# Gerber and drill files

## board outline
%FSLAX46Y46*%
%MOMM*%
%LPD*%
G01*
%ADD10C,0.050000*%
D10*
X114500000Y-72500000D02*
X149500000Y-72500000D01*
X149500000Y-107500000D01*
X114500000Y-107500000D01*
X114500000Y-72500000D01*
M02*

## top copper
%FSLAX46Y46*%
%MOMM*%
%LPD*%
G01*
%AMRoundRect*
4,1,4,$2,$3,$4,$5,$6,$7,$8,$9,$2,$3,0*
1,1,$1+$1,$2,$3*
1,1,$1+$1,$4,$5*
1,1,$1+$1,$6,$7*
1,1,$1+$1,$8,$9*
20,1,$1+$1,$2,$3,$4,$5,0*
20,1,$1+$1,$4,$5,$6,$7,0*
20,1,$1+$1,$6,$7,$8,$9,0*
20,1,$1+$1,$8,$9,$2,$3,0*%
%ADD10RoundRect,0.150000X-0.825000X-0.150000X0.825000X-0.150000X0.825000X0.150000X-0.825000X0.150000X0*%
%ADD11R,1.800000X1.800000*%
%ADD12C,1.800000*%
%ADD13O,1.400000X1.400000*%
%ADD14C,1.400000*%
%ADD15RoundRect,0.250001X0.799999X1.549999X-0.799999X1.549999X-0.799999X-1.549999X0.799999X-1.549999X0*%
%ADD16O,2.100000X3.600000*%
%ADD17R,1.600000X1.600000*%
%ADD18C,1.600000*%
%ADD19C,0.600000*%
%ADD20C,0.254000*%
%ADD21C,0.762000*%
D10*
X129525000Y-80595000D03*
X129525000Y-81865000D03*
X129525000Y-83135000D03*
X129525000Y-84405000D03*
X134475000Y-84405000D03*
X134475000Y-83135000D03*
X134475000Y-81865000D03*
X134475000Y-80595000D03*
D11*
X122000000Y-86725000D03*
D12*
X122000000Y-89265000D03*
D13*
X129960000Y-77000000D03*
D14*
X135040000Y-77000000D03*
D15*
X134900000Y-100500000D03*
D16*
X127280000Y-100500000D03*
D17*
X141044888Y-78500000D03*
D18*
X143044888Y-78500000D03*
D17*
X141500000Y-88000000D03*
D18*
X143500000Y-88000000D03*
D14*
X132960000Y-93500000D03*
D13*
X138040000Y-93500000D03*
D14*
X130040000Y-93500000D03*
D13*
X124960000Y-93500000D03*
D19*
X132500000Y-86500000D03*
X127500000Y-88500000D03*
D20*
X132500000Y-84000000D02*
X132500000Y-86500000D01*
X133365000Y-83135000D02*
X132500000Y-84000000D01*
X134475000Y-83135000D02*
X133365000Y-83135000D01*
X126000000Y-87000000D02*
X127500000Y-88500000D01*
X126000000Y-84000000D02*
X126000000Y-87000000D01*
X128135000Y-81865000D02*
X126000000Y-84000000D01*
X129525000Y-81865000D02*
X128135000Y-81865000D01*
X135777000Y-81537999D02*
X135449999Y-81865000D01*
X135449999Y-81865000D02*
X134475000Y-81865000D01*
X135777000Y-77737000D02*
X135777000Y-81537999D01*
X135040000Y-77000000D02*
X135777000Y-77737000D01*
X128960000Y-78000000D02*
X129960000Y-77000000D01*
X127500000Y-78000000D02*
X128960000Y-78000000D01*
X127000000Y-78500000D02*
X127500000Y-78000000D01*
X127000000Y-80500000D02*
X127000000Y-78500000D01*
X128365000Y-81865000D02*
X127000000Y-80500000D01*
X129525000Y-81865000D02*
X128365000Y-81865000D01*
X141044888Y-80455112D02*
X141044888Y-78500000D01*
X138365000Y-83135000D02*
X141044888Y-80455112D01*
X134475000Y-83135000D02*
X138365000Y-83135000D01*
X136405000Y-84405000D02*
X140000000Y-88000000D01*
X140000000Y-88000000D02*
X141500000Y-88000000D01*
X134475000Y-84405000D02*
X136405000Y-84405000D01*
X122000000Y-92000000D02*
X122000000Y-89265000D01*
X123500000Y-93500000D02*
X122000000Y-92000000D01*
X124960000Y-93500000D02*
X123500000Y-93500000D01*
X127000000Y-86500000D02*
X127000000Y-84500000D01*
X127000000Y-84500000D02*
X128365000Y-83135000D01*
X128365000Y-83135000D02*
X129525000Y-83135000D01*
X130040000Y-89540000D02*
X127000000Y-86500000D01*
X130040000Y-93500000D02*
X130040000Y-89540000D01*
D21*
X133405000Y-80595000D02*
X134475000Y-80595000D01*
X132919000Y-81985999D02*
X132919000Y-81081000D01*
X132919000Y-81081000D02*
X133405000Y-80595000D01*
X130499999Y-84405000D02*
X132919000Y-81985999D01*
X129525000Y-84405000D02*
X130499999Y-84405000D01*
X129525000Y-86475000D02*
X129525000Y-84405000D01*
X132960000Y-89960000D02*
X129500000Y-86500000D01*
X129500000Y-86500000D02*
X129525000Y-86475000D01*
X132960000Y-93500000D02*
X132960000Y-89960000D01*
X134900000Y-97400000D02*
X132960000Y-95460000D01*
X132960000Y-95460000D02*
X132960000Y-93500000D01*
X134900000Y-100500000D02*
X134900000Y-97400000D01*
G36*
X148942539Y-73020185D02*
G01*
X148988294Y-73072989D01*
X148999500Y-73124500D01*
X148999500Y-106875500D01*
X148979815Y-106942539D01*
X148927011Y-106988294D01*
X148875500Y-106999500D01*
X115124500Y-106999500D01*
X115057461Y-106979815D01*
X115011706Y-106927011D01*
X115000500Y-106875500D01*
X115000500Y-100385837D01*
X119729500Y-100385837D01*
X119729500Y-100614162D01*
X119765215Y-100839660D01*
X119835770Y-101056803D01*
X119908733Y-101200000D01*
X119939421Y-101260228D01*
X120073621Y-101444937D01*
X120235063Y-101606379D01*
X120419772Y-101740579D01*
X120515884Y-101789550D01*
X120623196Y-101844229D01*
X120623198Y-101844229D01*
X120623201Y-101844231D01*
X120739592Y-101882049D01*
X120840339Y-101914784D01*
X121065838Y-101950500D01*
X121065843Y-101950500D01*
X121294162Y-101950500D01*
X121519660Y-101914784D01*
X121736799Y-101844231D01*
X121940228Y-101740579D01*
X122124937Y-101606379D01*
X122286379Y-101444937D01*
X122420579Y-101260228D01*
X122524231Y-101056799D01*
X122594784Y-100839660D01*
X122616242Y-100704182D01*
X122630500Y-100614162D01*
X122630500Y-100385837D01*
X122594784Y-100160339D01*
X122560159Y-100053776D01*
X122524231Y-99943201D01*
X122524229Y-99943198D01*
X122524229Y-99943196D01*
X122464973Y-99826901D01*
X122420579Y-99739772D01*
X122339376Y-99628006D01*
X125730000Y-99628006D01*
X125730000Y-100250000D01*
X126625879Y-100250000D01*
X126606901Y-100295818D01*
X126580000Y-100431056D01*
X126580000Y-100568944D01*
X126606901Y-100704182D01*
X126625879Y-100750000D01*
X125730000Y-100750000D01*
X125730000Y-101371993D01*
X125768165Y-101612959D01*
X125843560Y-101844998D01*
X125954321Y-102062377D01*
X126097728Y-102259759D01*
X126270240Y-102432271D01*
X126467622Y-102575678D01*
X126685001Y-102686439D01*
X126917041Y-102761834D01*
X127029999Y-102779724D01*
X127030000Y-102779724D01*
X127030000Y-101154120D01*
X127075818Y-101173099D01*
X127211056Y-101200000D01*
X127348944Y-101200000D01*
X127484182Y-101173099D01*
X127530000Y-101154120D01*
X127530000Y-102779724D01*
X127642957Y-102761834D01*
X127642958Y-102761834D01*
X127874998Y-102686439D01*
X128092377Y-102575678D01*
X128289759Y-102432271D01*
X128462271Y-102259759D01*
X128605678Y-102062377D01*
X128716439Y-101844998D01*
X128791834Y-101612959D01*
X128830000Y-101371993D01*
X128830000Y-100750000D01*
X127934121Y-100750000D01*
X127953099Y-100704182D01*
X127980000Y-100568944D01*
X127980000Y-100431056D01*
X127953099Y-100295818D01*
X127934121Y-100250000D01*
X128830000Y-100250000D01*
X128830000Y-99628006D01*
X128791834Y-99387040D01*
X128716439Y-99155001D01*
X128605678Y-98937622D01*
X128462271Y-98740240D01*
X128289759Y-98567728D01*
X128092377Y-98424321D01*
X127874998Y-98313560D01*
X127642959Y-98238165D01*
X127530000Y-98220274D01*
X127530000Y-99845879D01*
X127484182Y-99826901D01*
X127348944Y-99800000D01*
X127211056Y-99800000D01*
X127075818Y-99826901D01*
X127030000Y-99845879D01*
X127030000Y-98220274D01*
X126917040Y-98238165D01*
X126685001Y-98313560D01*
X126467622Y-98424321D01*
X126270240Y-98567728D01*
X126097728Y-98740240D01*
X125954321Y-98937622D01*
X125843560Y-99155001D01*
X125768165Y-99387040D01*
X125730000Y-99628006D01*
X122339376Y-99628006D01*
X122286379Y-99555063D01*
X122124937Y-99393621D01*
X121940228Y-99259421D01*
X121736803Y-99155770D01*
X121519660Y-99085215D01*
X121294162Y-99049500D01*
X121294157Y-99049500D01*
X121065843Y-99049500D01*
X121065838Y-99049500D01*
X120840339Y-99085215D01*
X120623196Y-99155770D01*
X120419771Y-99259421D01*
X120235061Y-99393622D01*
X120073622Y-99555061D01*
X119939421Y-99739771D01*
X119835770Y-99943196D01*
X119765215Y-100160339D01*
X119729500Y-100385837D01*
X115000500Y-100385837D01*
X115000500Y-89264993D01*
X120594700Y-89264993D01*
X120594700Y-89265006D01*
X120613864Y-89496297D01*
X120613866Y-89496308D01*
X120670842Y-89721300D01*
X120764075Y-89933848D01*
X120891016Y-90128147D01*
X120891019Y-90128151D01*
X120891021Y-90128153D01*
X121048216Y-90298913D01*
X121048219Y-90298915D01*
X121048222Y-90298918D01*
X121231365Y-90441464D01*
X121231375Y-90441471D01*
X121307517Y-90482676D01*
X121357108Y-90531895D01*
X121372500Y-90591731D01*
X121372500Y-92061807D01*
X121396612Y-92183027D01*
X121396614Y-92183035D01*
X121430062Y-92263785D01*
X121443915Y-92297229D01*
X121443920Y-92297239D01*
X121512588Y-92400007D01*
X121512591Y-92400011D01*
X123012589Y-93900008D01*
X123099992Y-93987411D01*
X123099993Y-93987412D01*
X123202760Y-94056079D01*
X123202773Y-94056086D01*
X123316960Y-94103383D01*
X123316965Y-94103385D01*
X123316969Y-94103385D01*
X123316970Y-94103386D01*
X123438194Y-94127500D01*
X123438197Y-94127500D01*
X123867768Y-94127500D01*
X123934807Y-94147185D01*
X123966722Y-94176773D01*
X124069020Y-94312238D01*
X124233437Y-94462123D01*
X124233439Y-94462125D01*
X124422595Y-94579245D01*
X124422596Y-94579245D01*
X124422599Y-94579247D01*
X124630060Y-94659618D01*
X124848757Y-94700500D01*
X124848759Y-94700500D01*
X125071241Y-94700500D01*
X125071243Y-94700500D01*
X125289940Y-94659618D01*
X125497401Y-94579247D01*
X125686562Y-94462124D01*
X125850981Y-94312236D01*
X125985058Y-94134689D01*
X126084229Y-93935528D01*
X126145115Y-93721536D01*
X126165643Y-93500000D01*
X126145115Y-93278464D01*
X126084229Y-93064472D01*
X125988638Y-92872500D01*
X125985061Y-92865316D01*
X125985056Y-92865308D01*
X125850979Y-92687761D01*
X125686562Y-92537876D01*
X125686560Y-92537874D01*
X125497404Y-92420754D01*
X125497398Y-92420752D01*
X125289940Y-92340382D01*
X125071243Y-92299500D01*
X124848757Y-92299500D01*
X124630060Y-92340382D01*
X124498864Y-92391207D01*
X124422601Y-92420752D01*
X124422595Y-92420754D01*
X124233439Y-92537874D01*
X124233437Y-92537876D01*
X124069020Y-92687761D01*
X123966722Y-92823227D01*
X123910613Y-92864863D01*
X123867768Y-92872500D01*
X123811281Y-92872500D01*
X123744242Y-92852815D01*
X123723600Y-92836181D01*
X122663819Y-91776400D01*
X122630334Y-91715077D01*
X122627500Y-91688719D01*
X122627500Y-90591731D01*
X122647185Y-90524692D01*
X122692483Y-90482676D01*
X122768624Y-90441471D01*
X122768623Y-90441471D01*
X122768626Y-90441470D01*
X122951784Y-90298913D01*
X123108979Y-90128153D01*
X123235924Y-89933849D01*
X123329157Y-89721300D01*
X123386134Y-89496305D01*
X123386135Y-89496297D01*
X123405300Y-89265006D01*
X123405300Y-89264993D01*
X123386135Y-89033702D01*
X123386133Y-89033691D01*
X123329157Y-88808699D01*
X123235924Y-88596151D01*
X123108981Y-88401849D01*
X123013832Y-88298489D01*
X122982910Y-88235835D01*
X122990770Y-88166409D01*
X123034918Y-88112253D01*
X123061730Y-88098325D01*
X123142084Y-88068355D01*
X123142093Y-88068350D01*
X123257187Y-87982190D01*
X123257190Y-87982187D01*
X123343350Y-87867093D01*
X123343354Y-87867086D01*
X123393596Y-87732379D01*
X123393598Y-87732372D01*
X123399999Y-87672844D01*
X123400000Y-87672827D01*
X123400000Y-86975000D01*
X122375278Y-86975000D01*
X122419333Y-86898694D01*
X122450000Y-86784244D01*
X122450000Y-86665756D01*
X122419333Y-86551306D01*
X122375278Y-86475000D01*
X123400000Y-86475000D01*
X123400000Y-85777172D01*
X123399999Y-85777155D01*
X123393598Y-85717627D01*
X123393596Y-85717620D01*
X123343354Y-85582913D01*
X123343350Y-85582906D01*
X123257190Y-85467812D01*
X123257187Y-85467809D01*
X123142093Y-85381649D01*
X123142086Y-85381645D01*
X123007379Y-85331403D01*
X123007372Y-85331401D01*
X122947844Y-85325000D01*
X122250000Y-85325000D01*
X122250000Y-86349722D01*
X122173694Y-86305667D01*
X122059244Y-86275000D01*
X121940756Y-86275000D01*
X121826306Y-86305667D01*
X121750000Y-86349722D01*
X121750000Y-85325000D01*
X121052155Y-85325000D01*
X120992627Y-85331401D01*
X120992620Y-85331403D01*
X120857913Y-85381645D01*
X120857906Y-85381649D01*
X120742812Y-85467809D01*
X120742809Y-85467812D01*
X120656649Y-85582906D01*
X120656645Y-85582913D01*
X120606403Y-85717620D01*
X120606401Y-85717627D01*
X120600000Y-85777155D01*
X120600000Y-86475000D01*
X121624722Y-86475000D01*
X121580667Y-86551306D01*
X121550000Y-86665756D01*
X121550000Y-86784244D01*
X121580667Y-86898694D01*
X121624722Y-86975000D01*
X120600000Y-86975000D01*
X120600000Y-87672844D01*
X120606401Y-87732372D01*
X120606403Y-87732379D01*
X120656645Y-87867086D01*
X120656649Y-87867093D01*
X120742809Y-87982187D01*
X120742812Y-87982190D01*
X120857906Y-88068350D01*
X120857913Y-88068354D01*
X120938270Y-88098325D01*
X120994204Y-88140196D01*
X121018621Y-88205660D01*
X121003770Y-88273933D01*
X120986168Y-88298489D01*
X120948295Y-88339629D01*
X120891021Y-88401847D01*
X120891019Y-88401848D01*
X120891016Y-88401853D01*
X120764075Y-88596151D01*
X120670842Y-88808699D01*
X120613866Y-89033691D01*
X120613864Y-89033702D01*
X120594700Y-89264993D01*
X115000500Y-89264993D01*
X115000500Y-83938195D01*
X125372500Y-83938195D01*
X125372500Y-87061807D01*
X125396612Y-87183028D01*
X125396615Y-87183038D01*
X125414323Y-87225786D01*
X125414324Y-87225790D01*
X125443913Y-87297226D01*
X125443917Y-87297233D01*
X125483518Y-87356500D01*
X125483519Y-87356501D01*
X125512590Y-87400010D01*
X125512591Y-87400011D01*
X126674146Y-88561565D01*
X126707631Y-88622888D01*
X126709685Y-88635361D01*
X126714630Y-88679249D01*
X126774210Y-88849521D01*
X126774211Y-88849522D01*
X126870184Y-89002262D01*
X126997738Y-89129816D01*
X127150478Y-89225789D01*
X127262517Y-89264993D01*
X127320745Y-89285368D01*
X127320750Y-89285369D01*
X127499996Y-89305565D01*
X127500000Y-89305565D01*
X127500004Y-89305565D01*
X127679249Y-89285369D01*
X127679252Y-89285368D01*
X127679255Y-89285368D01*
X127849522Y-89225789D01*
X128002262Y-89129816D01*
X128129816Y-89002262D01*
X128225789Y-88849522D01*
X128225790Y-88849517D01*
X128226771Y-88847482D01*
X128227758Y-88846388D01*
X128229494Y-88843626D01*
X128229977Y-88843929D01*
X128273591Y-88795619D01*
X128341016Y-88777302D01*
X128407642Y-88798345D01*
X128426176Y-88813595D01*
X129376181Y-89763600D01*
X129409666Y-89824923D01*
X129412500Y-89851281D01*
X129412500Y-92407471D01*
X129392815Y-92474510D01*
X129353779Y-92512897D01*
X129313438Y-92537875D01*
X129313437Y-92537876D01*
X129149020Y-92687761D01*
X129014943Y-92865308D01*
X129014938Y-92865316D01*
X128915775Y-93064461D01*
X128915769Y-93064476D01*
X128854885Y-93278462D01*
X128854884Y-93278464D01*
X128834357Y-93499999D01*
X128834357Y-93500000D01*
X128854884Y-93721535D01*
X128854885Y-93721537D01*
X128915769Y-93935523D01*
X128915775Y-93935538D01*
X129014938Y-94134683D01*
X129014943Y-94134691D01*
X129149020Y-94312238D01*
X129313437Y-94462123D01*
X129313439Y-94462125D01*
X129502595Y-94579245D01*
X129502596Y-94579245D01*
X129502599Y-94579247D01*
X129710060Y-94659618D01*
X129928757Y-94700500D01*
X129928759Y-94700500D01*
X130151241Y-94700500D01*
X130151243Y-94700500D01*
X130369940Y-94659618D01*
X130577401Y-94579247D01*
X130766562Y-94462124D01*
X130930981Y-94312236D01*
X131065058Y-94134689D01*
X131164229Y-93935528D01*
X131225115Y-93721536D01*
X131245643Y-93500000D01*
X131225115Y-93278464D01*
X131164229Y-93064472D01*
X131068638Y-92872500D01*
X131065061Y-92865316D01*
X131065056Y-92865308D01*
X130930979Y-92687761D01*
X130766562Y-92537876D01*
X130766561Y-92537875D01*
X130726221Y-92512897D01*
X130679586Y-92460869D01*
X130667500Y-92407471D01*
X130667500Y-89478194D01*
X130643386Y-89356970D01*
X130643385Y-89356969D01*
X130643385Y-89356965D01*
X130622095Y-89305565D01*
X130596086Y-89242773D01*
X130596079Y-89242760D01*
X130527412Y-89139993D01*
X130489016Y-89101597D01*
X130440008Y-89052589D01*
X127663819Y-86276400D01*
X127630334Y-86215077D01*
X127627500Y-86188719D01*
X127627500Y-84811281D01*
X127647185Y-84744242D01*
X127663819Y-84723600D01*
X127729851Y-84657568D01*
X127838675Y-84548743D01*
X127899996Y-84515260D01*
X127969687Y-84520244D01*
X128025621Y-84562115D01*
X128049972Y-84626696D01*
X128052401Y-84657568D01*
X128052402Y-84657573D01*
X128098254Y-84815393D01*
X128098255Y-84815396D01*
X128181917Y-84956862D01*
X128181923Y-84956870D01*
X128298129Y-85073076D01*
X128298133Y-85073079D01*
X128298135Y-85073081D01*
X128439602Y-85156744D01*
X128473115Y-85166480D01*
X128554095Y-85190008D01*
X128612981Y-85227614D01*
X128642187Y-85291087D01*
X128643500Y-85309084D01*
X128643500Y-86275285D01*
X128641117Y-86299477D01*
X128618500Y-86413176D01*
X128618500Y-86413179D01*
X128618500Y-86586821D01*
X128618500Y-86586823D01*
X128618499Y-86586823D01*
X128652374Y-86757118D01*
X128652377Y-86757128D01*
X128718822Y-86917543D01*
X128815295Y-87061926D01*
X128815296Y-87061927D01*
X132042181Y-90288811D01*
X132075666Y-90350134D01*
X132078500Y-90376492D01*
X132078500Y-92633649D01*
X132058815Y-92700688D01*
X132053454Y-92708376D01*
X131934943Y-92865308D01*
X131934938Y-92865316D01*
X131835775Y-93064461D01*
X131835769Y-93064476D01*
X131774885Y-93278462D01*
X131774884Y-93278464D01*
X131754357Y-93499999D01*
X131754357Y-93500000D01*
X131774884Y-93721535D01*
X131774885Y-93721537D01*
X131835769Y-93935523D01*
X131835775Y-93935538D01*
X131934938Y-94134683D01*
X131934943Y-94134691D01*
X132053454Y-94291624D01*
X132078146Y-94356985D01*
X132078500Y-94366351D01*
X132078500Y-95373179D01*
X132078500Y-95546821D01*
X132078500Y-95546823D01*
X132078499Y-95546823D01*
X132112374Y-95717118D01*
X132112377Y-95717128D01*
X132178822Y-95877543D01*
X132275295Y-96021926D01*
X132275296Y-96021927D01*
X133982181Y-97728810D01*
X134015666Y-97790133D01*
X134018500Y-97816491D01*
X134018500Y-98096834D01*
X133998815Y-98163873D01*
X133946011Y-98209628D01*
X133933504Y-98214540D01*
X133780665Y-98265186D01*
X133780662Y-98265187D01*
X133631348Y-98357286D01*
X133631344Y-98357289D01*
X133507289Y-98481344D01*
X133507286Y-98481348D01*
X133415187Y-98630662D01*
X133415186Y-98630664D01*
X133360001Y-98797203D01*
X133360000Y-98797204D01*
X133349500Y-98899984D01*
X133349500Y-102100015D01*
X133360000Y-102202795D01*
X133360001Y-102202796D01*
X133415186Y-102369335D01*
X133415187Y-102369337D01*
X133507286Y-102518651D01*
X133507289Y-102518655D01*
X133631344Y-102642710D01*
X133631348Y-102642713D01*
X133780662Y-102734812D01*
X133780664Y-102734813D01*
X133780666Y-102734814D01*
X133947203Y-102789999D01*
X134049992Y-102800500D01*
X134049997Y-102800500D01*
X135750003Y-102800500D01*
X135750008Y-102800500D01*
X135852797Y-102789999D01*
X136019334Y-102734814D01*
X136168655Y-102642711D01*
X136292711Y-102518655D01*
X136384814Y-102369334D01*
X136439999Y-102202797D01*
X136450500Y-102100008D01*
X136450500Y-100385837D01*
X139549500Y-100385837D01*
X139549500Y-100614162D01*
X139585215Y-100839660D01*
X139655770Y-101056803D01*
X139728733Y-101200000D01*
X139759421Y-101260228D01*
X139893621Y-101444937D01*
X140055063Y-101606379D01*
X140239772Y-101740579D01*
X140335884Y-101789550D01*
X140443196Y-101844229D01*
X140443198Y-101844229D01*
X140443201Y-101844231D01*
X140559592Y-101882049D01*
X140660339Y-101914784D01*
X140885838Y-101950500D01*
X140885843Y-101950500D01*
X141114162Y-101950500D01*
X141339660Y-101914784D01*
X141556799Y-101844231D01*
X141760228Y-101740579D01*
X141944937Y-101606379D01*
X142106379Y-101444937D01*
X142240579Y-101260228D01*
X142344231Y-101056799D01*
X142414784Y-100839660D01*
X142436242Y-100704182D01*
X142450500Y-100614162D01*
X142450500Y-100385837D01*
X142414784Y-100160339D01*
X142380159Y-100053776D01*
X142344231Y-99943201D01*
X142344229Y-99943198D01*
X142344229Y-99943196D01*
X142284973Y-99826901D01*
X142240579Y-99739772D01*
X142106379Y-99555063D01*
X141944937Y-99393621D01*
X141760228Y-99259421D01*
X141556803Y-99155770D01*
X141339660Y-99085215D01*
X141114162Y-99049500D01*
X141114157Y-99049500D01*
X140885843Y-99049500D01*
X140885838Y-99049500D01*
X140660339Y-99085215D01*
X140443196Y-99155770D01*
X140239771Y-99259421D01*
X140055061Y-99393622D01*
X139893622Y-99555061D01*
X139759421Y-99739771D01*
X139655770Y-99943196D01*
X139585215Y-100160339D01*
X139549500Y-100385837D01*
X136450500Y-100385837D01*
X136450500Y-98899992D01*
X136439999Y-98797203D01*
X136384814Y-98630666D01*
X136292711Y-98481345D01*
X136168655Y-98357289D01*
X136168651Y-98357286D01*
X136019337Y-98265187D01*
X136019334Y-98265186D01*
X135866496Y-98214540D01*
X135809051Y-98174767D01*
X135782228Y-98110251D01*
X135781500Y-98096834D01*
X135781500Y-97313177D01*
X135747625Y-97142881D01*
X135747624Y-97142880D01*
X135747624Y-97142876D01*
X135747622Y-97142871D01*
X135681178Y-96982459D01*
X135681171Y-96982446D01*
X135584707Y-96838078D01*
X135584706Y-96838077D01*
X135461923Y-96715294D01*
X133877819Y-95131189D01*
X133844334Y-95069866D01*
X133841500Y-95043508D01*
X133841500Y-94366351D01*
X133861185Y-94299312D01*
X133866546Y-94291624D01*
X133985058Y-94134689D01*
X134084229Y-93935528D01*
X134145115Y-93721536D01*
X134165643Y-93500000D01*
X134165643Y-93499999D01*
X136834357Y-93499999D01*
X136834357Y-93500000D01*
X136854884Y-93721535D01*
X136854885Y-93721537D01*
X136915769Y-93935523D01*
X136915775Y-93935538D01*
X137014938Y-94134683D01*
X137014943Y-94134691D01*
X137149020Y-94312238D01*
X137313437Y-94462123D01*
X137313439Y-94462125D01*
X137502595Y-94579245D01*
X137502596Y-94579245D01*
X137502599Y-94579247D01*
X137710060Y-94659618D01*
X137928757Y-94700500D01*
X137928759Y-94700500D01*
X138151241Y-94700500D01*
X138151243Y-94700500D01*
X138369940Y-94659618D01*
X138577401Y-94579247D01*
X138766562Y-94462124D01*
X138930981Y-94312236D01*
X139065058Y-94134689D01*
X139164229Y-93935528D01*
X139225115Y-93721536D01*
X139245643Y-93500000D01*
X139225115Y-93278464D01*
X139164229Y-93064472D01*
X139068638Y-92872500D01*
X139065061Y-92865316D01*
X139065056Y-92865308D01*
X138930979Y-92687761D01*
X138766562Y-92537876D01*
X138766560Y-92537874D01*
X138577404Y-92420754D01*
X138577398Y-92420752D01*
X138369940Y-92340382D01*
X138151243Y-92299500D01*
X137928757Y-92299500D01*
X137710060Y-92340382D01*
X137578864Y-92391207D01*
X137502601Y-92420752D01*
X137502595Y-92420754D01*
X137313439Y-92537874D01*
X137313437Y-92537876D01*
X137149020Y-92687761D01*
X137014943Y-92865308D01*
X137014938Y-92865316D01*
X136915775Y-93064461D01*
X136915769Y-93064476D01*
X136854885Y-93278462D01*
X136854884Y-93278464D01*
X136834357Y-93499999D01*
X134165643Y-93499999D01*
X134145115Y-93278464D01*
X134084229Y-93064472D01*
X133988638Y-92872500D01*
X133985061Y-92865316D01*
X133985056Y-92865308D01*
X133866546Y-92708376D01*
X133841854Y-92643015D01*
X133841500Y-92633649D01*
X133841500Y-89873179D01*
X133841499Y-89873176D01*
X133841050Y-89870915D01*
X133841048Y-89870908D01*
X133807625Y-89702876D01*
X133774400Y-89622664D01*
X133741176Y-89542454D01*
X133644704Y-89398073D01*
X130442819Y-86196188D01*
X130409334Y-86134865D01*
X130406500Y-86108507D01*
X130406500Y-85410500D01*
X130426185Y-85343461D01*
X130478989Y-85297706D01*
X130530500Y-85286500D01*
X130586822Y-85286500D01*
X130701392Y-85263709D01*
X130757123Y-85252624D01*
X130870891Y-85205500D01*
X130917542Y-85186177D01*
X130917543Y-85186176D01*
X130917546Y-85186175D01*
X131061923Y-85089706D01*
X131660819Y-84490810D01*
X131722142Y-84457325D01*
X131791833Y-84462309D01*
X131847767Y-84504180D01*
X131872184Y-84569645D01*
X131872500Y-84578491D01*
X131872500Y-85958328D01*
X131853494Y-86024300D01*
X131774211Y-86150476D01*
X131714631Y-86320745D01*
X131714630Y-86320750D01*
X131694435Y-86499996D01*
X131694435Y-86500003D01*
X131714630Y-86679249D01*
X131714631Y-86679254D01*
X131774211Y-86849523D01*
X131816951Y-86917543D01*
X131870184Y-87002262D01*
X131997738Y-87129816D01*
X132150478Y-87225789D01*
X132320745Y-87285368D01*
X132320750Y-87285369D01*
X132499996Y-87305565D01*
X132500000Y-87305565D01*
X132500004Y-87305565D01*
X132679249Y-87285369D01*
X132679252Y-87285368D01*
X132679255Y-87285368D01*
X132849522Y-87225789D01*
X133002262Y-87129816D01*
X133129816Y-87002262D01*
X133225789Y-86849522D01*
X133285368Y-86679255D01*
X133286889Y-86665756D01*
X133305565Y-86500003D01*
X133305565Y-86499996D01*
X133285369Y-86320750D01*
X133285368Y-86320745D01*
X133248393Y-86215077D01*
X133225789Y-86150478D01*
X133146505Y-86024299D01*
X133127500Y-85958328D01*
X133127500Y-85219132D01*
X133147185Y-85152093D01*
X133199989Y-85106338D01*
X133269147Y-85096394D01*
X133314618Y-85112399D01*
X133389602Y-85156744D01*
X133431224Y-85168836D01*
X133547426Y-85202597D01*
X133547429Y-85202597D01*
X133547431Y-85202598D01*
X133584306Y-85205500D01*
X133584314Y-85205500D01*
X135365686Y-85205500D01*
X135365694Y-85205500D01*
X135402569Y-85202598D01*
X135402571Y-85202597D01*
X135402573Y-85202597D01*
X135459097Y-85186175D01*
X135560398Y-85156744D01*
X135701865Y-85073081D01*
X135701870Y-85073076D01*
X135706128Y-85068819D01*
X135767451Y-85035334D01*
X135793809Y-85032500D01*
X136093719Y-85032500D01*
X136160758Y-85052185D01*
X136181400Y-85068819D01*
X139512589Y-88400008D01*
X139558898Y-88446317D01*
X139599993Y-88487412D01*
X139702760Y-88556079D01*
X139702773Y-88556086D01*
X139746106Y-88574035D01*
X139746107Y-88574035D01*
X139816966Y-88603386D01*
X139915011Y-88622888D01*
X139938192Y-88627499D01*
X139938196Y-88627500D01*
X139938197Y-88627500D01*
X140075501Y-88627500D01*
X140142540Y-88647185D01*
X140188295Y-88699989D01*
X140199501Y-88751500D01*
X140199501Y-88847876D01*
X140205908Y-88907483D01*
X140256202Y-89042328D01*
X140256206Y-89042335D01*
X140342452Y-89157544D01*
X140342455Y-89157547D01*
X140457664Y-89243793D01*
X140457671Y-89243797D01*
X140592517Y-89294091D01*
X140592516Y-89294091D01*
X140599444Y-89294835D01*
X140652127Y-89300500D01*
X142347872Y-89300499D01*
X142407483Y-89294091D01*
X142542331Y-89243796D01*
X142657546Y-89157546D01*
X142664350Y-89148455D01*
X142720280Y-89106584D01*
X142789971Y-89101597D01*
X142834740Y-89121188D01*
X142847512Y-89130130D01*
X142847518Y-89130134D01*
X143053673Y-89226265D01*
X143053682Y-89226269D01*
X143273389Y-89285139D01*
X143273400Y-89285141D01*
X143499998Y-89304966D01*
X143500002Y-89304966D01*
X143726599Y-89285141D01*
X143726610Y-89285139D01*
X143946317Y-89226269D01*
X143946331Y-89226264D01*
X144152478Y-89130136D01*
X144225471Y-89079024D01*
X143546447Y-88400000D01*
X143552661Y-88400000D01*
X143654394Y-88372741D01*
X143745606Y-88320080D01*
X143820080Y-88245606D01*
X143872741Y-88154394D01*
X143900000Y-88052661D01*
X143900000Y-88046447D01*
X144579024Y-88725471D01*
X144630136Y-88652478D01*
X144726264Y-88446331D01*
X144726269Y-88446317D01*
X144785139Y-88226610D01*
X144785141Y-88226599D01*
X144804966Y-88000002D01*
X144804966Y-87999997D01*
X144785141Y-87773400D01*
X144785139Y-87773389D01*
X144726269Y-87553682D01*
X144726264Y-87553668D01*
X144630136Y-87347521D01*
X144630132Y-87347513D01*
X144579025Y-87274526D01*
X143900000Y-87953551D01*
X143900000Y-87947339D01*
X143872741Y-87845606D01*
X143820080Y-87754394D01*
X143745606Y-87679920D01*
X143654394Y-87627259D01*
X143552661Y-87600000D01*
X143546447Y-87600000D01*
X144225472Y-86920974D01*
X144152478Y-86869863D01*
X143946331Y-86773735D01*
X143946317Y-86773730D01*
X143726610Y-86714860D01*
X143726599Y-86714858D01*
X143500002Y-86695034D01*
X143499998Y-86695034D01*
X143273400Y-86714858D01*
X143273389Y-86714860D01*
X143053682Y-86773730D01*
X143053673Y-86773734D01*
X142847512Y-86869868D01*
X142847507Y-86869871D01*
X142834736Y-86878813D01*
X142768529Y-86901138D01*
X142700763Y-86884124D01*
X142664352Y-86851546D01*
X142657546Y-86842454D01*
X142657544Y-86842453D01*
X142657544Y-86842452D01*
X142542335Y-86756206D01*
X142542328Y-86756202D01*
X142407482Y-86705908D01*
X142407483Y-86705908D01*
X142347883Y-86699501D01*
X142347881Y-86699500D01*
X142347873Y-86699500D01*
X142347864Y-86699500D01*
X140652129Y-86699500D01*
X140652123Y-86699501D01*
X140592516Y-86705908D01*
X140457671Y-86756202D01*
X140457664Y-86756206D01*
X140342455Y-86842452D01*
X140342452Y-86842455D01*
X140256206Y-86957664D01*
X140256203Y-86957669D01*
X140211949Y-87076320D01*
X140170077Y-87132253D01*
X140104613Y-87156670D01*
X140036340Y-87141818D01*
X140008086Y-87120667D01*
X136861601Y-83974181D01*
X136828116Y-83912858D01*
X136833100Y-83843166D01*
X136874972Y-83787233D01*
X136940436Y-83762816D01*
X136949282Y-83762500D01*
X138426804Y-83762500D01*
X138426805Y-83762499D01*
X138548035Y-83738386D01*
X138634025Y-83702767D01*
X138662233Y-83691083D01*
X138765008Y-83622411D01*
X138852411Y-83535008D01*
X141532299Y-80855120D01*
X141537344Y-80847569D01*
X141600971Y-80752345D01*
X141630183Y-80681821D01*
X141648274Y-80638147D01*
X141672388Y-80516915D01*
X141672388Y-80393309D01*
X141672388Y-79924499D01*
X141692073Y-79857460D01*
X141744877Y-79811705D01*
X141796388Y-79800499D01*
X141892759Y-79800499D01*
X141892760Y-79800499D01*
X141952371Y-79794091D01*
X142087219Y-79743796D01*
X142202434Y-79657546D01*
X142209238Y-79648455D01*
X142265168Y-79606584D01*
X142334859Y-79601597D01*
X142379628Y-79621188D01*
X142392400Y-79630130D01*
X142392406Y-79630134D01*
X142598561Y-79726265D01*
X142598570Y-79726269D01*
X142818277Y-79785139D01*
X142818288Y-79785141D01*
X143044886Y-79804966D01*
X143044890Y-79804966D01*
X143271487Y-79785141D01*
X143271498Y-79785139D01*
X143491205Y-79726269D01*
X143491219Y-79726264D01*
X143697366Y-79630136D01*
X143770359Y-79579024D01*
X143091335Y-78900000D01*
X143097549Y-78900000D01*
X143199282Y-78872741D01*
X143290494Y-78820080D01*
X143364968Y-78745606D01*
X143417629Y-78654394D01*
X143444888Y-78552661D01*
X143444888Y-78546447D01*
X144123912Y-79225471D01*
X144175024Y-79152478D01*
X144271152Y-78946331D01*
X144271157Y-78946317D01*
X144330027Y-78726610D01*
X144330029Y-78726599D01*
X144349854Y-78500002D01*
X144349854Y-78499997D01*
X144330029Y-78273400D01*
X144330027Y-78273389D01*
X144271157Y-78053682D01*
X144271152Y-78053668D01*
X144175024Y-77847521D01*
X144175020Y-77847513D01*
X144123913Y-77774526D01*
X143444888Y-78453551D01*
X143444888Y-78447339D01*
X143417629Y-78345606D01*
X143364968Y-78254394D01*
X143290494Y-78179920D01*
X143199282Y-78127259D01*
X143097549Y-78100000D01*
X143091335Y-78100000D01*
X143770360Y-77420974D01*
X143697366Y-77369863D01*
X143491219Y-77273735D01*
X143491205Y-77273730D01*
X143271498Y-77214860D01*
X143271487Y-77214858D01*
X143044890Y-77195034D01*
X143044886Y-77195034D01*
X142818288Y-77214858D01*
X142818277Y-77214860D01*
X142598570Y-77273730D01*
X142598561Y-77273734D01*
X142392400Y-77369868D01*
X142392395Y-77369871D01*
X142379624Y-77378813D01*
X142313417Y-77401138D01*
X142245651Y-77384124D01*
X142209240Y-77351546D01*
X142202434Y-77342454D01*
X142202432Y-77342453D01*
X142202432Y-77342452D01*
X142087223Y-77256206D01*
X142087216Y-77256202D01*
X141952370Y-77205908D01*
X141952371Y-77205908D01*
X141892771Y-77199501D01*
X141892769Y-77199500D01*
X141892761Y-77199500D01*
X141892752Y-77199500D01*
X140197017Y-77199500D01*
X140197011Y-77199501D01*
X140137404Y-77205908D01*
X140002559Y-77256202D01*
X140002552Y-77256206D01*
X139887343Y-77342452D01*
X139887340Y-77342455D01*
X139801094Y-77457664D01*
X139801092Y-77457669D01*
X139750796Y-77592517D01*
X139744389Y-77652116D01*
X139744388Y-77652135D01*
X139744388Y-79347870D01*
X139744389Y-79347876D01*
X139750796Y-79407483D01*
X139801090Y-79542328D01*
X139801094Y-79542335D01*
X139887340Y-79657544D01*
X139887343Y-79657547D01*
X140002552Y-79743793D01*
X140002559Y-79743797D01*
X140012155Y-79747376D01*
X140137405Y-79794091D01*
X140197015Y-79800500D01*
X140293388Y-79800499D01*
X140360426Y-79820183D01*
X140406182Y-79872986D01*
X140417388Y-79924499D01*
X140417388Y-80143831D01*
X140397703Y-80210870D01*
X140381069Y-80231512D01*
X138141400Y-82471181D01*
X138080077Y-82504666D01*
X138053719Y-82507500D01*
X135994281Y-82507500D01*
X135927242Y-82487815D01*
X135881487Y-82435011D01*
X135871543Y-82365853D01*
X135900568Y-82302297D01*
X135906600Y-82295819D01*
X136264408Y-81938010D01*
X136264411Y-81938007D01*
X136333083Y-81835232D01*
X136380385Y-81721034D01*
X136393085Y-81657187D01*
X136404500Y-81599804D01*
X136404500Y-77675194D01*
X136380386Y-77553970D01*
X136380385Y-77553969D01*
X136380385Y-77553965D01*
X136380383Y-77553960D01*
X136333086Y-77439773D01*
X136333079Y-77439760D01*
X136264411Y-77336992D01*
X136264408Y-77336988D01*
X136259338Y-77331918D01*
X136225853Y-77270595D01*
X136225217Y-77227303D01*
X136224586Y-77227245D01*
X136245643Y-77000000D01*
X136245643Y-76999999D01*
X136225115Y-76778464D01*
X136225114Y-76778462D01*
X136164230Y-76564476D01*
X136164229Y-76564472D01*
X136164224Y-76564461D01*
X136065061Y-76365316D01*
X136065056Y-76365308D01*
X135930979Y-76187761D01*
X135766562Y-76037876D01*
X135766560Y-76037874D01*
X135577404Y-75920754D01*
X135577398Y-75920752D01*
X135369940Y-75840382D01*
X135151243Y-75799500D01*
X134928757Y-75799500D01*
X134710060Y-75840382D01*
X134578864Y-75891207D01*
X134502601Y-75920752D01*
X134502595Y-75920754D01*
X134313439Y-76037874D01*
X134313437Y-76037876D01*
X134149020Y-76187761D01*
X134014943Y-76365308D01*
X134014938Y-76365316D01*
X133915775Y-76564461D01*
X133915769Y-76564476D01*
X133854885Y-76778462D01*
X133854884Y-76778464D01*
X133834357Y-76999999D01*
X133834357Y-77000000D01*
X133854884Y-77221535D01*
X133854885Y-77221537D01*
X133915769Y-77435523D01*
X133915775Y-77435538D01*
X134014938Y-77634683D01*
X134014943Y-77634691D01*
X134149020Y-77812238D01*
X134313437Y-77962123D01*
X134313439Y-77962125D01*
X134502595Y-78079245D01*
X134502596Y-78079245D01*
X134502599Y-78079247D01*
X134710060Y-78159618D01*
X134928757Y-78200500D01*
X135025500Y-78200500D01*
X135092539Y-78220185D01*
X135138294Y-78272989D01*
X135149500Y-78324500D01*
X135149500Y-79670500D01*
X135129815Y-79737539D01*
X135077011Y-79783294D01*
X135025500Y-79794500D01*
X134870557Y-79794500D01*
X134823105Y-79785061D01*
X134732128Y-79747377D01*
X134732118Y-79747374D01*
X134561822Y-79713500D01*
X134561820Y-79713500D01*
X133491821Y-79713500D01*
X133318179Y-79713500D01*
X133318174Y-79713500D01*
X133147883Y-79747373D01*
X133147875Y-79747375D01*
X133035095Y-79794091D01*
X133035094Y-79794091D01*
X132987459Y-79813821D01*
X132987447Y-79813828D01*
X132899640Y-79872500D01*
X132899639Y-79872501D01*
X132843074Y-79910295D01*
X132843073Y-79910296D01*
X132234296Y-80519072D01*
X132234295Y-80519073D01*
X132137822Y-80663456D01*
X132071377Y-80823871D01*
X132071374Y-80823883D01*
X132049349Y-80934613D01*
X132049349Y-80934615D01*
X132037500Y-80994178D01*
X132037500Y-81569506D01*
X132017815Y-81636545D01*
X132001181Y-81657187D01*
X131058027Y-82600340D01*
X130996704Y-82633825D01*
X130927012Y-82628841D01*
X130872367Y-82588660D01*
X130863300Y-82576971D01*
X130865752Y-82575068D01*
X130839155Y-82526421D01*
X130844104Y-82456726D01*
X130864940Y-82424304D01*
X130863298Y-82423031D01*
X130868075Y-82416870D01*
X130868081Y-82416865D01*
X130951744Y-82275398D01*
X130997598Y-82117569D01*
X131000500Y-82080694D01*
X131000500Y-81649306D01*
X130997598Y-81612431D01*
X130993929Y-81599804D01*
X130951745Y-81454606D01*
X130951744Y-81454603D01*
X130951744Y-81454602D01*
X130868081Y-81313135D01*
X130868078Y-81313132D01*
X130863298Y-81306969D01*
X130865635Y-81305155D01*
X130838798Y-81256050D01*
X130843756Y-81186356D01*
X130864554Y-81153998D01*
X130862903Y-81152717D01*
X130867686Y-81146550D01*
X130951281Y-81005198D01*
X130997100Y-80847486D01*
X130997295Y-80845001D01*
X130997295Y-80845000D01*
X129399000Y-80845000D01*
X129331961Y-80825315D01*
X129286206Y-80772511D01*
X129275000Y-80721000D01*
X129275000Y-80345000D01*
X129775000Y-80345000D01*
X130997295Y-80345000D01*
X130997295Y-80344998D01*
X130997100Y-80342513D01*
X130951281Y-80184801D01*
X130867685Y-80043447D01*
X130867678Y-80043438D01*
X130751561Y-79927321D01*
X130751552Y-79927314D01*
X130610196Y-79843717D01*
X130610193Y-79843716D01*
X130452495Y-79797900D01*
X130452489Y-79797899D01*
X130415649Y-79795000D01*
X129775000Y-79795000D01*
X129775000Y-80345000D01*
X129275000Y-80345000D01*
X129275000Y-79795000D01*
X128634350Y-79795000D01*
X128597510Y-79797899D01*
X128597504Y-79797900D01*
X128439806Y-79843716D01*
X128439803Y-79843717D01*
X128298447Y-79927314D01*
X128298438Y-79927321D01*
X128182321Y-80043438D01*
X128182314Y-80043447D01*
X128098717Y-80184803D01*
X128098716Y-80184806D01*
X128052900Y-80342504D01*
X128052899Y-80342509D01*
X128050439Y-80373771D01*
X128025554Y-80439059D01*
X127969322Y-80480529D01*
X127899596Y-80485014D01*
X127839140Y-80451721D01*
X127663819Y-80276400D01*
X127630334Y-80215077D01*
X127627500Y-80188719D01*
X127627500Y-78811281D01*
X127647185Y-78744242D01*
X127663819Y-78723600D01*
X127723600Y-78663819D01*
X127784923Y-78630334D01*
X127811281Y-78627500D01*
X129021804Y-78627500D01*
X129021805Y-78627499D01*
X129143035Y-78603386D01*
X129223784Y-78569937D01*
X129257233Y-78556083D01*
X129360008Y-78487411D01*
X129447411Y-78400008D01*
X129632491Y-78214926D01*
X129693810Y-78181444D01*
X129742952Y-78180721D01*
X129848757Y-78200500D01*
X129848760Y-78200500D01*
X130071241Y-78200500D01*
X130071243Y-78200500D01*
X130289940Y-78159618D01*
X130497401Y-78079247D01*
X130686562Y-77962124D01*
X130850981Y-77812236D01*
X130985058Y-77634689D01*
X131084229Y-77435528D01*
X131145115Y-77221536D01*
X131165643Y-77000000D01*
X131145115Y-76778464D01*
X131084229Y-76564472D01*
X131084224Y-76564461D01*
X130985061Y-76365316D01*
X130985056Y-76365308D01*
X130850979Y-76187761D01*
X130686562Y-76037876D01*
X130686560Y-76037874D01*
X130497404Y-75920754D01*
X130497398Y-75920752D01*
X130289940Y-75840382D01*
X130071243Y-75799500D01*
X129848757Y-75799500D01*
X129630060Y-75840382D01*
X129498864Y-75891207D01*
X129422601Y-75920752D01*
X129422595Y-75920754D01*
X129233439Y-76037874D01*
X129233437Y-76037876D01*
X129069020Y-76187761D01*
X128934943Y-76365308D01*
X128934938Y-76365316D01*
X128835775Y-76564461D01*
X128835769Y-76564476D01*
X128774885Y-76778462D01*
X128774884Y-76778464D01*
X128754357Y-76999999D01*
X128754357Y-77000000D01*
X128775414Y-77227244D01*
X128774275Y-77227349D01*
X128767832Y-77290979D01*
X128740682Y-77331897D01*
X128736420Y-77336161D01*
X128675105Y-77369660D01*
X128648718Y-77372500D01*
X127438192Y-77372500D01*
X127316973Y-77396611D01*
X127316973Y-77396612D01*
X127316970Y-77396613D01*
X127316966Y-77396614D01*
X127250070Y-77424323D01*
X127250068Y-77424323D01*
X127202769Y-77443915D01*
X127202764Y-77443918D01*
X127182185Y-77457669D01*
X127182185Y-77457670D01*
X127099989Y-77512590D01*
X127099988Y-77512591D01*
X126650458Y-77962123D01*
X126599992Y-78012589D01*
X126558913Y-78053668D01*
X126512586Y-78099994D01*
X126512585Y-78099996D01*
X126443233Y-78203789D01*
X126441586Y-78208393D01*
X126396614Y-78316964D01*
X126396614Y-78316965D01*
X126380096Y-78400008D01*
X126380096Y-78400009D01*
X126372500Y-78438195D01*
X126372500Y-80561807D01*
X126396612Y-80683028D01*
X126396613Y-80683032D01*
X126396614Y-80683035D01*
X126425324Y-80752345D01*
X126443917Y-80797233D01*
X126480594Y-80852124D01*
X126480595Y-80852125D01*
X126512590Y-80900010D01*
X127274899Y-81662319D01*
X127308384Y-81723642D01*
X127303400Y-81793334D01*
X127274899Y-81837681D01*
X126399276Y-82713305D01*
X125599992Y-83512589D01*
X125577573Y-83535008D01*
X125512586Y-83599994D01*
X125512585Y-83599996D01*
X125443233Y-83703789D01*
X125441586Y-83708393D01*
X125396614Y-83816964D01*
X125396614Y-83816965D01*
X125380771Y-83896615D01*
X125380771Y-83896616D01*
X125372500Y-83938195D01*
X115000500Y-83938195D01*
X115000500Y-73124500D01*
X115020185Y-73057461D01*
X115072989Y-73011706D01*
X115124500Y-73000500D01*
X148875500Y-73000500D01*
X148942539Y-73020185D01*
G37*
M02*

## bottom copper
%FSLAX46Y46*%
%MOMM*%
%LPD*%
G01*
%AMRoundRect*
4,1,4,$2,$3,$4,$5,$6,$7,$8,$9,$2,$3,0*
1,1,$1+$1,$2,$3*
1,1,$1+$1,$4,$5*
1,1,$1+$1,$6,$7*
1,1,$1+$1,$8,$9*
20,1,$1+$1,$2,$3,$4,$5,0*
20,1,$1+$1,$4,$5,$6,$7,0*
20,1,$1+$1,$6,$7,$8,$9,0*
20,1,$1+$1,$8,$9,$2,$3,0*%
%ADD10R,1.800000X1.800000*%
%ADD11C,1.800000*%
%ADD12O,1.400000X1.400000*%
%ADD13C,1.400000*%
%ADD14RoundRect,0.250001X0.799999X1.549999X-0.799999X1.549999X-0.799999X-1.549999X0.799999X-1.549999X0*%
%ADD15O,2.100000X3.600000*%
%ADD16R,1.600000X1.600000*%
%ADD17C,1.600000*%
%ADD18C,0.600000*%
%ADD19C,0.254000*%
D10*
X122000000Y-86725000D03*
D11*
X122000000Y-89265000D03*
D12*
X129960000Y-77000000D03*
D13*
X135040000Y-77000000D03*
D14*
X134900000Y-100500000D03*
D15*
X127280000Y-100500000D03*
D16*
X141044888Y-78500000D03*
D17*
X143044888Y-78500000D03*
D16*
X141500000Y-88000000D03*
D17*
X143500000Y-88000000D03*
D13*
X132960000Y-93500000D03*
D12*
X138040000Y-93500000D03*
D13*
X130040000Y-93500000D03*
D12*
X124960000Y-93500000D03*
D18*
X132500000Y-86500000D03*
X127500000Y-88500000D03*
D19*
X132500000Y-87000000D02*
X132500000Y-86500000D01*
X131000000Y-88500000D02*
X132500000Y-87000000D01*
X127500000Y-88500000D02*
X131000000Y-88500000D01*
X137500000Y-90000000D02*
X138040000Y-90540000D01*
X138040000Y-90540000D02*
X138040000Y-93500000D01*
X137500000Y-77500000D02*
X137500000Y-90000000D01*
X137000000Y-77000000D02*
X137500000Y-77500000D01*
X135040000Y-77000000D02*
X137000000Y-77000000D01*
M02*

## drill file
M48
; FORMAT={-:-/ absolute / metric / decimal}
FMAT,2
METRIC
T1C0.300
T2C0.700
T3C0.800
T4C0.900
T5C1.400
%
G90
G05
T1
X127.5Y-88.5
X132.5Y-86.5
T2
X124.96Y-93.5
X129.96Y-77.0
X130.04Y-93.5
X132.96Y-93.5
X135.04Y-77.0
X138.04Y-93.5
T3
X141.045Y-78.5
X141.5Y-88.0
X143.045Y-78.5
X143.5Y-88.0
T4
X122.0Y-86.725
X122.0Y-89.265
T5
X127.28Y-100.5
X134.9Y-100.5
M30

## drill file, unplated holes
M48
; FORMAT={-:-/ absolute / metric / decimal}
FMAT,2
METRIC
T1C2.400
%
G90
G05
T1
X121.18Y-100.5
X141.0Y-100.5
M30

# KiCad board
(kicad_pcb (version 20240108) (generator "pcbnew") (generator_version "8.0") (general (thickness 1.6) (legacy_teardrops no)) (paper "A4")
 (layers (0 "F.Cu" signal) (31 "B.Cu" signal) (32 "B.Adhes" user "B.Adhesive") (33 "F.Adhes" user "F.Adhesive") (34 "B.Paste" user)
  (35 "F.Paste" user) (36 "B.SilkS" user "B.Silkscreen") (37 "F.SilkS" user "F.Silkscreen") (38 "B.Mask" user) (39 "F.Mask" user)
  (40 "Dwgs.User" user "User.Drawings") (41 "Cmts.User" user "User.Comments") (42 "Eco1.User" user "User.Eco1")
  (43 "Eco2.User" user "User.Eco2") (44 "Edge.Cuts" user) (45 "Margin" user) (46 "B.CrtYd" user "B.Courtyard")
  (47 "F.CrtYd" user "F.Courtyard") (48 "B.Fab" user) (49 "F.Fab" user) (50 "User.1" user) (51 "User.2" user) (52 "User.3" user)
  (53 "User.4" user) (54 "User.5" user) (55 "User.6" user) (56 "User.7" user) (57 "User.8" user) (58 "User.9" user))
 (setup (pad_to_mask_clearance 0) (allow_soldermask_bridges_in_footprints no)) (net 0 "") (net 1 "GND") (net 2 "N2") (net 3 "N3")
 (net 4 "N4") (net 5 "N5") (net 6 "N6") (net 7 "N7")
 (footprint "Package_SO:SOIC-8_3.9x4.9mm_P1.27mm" (layer "F.Cu") (at 132 82.5)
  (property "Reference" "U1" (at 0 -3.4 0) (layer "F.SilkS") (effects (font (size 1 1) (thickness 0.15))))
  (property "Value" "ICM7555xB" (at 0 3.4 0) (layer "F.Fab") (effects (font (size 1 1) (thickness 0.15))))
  (pad "1" smd roundrect (at -2.475 -1.905) (size 1.95 0.6) (layers "F.Cu" "F.Paste" "F.Mask") (roundrect_rratio 0.25) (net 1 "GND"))
  (pad "2" smd roundrect (at -2.475 -0.635) (size 1.95 0.6) (layers "F.Cu" "F.Paste" "F.Mask") (roundrect_rratio 0.25) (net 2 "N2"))
  (pad "3" smd roundrect (at -2.475 0.635) (size 1.95 0.6) (layers "F.Cu" "F.Paste" "F.Mask") (roundrect_rratio 0.25) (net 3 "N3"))
  (pad "4" smd roundrect (at -2.475 1.905) (size 1.95 0.6) (layers "F.Cu" "F.Paste" "F.Mask") (roundrect_rratio 0.25) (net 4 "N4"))
  (pad "5" smd roundrect (at 2.475 1.905) (size 1.95 0.6) (layers "F.Cu" "F.Paste" "F.Mask") (roundrect_rratio 0.25) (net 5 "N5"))
  (pad "6" smd roundrect (at 2.475 0.635) (size 1.95 0.6) (layers "F.Cu" "F.Paste" "F.Mask") (roundrect_rratio 0.25) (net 2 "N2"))
  (pad "7" smd roundrect (at 2.475 -0.635) (size 1.95 0.6) (layers "F.Cu" "F.Paste" "F.Mask") (roundrect_rratio 0.25) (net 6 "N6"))
  (pad "8" smd roundrect (at 2.475 -1.905) (size 1.95 0.6) (layers "F.Cu" "F.Paste" "F.Mask") (roundrect_rratio 0.25) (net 4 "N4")))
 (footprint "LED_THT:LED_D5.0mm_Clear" (layer "F.Cu") (at 122 86.725 -90)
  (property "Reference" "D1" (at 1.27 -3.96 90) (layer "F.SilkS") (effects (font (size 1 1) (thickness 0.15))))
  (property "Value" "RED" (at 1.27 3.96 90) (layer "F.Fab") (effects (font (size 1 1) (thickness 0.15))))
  (pad "1" thru_hole rect (at 0 0 270) (size 1.8 1.8) (drill 0.9) (layers "*.Cu" "*.Mask") (remove_unused_layers no) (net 1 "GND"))
  (pad "2" thru_hole circle (at 2.54 0 270) (size 1.8 1.8) (drill 0.9) (layers "*.Cu" "*.Mask") (remove_unused_layers no) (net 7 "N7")))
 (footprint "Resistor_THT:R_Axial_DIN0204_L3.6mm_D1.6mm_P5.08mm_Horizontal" (layer "F.Cu") (at 135.04 77 180)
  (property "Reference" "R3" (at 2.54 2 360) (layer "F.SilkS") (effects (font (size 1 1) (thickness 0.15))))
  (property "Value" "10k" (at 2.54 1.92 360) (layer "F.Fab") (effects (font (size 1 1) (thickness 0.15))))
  (pad "1" thru_hole circle (at 0 0 180) (size 1.4 1.4) (drill 0.7) (layers "*.Cu" "*.Mask") (remove_unused_layers no) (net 6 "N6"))
  (pad "2" thru_hole oval (at 5.08 0 180) (size 1.4 1.4) (drill 0.7) (layers "*.Cu" "*.Mask") (remove_unused_layers no) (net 2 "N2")))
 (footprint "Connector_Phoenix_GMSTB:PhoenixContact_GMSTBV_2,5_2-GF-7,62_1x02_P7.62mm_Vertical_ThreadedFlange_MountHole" (layer "F.Cu")
  (at 134.9 100.5 180)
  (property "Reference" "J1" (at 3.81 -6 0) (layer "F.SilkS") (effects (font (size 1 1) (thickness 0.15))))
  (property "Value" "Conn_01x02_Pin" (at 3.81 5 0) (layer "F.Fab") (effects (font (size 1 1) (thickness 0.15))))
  (pad "" np_thru_hole circle (at -6.1 0 180) (size 2.4 2.4) (drill 2.4) (layers "*.Cu" "*.Mask"))
  (pad "" np_thru_hole circle (at 13.72 0 180) (size 2.4 2.4) (drill 2.4) (layers "*.Cu" "*.Mask"))
  (pad "1" thru_hole roundrect (at 0 0 180) (size 2.1 3.6) (drill 1.4) (layers "*.Cu" "*.Mask") (remove_unused_layers no)
   (roundrect_rratio 0.119048) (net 4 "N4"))
  (pad "2" thru_hole oval (at 7.62 0 180) (size 2.1 3.6) (drill 1.4) (layers "*.Cu" "*.Mask") (remove_unused_layers no) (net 1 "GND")))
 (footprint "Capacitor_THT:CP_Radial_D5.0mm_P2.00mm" (layer "F.Cu") (at 141.044888 78.5)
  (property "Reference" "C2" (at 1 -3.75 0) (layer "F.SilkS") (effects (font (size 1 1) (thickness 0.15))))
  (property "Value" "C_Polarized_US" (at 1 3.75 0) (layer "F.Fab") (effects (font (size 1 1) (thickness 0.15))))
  (pad "1" thru_hole rect (at 0 0) (size 1.6 1.6) (drill 0.8) (layers "*.Cu" "*.Mask") (remove_unused_layers no) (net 2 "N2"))
  (pad "2" thru_hole circle (at 2 0) (size 1.6 1.6) (drill 0.8) (layers "*.Cu" "*.Mask") (remove_unused_layers no) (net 1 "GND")))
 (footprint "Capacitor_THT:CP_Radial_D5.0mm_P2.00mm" (layer "F.Cu") (at 141.5 88)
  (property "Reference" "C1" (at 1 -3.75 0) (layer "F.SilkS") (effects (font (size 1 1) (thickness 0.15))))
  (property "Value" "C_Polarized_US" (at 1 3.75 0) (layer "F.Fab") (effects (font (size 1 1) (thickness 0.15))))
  (pad "1" thru_hole rect (at 0 0) (size 1.6 1.6) (drill 0.8) (layers "*.Cu" "*.Mask") (remove_unused_layers no) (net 5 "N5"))
  (pad "2" thru_hole circle (at 2 0) (size 1.6 1.6) (drill 0.8) (layers "*.Cu" "*.Mask") (remove_unused_layers no) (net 1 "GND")))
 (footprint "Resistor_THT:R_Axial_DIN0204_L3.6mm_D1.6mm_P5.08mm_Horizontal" (layer "F.Cu") (at 132.96 93.5)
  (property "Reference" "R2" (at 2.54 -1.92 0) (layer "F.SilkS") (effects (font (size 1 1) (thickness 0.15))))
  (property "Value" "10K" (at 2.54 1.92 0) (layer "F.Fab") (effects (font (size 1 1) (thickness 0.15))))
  (pad "1" thru_hole circle (at 0 0) (size 1.4 1.4) (drill 0.7) (layers "*.Cu" "*.Mask") (remove_unused_layers no) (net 4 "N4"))
  (pad "2" thru_hole oval (at 5.08 0) (size 1.4 1.4) (drill 0.7) (layers "*.Cu" "*.Mask") (remove_unused_layers no) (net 6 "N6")))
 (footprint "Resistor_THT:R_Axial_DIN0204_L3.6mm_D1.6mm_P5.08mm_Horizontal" (layer "F.Cu") (at 130.04 93.5 180)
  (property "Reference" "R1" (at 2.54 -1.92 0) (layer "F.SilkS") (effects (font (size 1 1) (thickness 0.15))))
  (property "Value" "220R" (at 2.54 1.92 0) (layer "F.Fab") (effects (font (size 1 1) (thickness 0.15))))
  (pad "1" thru_hole circle (at 0 0 180) (size 1.4 1.4) (drill 0.7) (layers "*.Cu" "*.Mask") (remove_unused_layers no) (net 3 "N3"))
  (pad "2" thru_hole oval (at 5.08 0 180) (size 1.4 1.4) (drill 0.7) (layers "*.Cu" "*.Mask") (remove_unused_layers no) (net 7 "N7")))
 (gr_rect (start 114.5 72.5) (end 149.5 107.5) (stroke (width 0.05) (type default)) (fill none) (layer "Edge.Cuts"))
 (segment (start 136.405 84.405) (end 140 88) (width 0.254) (layer "F.Cu") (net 5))
 (segment (start 140 88) (end 141.5 88) (width 0.254) (layer "F.Cu") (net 5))
 (segment (start 134.475 84.405) (end 136.405 84.405) (width 0.254) (layer "F.Cu") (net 5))
 (segment (start 127.5 78) (end 128.96 78) (width 0.254) (layer "F.Cu") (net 2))
 (segment (start 126 84) (end 126 87) (width 0.254) (layer "F.Cu") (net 2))
 (segment (start 134.475 83.135) (end 133.365 83.135) (width 0.254) (layer "F.Cu") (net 2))
 (segment (start 141.044888 80.455112) (end 141.044888 78.5) (width 0.254) (layer "F.Cu") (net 2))
 (segment (start 128.96 78) (end 129.96 77) (width 0.254) (layer "F.Cu") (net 2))
 (segment (start 127 80.5) (end 127 78.5) (width 0.254) (layer "F.Cu") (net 2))
 (segment (start 126 87) (end 127.5 88.5) (width 0.254) (layer "F.Cu") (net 2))
 (segment (start 129.525 81.865) (end 128.135 81.865) (width 0.254) (layer "F.Cu") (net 2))
 (segment (start 132.5 84) (end 132.5 86.5) (width 0.254) (layer "F.Cu") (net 2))
 (segment (start 127 78.5) (end 127.5 78) (width 0.254) (layer "F.Cu") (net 2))
 (segment (start 133.365 83.135) (end 132.5 84) (width 0.254) (layer "F.Cu") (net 2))
 (segment (start 128.365 81.865) (end 127 80.5) (width 0.254) (layer "F.Cu") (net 2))
 (segment (start 129.525 81.865) (end 128.365 81.865) (width 0.254) (layer "F.Cu") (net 2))
 (segment (start 134.475 83.135) (end 138.365 83.135) (width 0.254) (layer "F.Cu") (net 2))
 (segment (start 138.365 83.135) (end 141.044888 80.455112) (width 0.254) (layer "F.Cu") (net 2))
 (segment (start 128.135 81.865) (end 126 84) (width 0.254) (layer "F.Cu") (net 2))
 (via (at 132.5 86.5) (size 0.6) (drill 0.3) (layers "F.Cu" "B.Cu") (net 2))
 (via (at 127.5 88.5) (size 0.6) (drill 0.3) (layers "F.Cu" "B.Cu") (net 2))
 (segment (start 132.5 87) (end 132.5 86.5) (width 0.254) (layer "B.Cu") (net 2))
 (segment (start 131 88.5) (end 132.5 87) (width 0.254) (layer "B.Cu") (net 2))
 (segment (start 127.5 88.5) (end 131 88.5) (width 0.254) (layer "B.Cu") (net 2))
 (segment (start 122 92) (end 122 89.265) (width 0.254) (layer "F.Cu") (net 7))
 (segment (start 124.96 93.5) (end 123.5 93.5) (width 0.254) (layer "F.Cu") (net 7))
 (segment (start 123.5 93.5) (end 122 92) (width 0.254) (layer "F.Cu") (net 7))
 (segment (start 132.919 81.985999) (end 132.919 81.081) (width 0.762) (layer "F.Cu") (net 4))
 (segment (start 132.96 89.96) (end 129.5 86.5) (width 0.762) (layer "F.Cu") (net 4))
 (segment (start 133.405 80.595) (end 134.475 80.595) (width 0.762) (layer "F.Cu") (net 4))
 (segment (start 129.525 84.405) (end 130.499999 84.405) (width 0.762) (layer "F.Cu") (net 4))
 (segment (start 132.96 93.5) (end 132.96 89.96) (width 0.762) (layer "F.Cu") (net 4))
 (segment (start 132.919 81.081) (end 133.405 80.595) (width 0.762) (layer "F.Cu") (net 4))
 (segment (start 129.5 86.5) (end 129.525 86.475) (width 0.762) (layer "F.Cu") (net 4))
 (segment (start 129.525 86.475) (end 129.525 84.405) (width 0.762) (layer "F.Cu") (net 4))
 (segment (start 134.9 97.4) (end 132.96 95.46) (width 0.762) (layer "F.Cu") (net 4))
 (segment (start 134.9 100.5) (end 134.9 97.4) (width 0.762) (layer "F.Cu") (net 4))
 (segment (start 130.499999 84.405) (end 132.919 81.985999) (width 0.762) (layer "F.Cu") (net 4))
 (segment (start 132.96 95.46) (end 132.96 93.5) (width 0.762) (layer "F.Cu") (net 4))
 (segment (start 127 84.5) (end 128.365 83.135) (width 0.254) (layer "F.Cu") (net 3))
 (segment (start 130.04 89.54) (end 127 86.5) (width 0.254) (layer "F.Cu") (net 3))
 (segment (start 130.04 93.5) (end 130.04 89.54) (width 0.254) (layer "F.Cu") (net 3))
 (segment (start 127 86.5) (end 127 84.5) (width 0.254) (layer "F.Cu") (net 3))
 (segment (start 128.365 83.135) (end 129.525 83.135) (width 0.254) (layer "F.Cu") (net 3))
 (segment (start 135.777 77.737) (end 135.777 81.537999) (width 0.254) (layer "F.Cu") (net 6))
 (segment (start 135.449999 81.865) (end 134.475 81.865) (width 0.254) (layer "F.Cu") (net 6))
 (segment (start 135.777 81.537999) (end 135.449999 81.865) (width 0.254) (layer "F.Cu") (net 6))
 (segment (start 135.04 77) (end 135.777 77.737) (width 0.254) (layer "F.Cu") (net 6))
 (segment (start 137.5 77.5) (end 137.5 90) (width 0.254) (layer "B.Cu") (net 6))
 (segment (start 138.04 90.54) (end 138.04 93.5) (width 0.254) (layer "B.Cu") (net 6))
 (segment (start 137 77) (end 137.5 77.5) (width 0.254) (layer "B.Cu") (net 6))
 (segment (start 137.5 90) (end 138.04 90.54) (width 0.254) (layer "B.Cu") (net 6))
 (segment (start 135.04 77) (end 137 77) (width 0.254) (layer "B.Cu") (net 6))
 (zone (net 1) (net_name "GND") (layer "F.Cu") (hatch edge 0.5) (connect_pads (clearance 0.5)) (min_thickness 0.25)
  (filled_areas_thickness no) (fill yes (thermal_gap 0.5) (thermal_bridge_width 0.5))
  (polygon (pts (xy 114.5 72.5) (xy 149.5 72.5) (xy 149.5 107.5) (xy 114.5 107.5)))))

